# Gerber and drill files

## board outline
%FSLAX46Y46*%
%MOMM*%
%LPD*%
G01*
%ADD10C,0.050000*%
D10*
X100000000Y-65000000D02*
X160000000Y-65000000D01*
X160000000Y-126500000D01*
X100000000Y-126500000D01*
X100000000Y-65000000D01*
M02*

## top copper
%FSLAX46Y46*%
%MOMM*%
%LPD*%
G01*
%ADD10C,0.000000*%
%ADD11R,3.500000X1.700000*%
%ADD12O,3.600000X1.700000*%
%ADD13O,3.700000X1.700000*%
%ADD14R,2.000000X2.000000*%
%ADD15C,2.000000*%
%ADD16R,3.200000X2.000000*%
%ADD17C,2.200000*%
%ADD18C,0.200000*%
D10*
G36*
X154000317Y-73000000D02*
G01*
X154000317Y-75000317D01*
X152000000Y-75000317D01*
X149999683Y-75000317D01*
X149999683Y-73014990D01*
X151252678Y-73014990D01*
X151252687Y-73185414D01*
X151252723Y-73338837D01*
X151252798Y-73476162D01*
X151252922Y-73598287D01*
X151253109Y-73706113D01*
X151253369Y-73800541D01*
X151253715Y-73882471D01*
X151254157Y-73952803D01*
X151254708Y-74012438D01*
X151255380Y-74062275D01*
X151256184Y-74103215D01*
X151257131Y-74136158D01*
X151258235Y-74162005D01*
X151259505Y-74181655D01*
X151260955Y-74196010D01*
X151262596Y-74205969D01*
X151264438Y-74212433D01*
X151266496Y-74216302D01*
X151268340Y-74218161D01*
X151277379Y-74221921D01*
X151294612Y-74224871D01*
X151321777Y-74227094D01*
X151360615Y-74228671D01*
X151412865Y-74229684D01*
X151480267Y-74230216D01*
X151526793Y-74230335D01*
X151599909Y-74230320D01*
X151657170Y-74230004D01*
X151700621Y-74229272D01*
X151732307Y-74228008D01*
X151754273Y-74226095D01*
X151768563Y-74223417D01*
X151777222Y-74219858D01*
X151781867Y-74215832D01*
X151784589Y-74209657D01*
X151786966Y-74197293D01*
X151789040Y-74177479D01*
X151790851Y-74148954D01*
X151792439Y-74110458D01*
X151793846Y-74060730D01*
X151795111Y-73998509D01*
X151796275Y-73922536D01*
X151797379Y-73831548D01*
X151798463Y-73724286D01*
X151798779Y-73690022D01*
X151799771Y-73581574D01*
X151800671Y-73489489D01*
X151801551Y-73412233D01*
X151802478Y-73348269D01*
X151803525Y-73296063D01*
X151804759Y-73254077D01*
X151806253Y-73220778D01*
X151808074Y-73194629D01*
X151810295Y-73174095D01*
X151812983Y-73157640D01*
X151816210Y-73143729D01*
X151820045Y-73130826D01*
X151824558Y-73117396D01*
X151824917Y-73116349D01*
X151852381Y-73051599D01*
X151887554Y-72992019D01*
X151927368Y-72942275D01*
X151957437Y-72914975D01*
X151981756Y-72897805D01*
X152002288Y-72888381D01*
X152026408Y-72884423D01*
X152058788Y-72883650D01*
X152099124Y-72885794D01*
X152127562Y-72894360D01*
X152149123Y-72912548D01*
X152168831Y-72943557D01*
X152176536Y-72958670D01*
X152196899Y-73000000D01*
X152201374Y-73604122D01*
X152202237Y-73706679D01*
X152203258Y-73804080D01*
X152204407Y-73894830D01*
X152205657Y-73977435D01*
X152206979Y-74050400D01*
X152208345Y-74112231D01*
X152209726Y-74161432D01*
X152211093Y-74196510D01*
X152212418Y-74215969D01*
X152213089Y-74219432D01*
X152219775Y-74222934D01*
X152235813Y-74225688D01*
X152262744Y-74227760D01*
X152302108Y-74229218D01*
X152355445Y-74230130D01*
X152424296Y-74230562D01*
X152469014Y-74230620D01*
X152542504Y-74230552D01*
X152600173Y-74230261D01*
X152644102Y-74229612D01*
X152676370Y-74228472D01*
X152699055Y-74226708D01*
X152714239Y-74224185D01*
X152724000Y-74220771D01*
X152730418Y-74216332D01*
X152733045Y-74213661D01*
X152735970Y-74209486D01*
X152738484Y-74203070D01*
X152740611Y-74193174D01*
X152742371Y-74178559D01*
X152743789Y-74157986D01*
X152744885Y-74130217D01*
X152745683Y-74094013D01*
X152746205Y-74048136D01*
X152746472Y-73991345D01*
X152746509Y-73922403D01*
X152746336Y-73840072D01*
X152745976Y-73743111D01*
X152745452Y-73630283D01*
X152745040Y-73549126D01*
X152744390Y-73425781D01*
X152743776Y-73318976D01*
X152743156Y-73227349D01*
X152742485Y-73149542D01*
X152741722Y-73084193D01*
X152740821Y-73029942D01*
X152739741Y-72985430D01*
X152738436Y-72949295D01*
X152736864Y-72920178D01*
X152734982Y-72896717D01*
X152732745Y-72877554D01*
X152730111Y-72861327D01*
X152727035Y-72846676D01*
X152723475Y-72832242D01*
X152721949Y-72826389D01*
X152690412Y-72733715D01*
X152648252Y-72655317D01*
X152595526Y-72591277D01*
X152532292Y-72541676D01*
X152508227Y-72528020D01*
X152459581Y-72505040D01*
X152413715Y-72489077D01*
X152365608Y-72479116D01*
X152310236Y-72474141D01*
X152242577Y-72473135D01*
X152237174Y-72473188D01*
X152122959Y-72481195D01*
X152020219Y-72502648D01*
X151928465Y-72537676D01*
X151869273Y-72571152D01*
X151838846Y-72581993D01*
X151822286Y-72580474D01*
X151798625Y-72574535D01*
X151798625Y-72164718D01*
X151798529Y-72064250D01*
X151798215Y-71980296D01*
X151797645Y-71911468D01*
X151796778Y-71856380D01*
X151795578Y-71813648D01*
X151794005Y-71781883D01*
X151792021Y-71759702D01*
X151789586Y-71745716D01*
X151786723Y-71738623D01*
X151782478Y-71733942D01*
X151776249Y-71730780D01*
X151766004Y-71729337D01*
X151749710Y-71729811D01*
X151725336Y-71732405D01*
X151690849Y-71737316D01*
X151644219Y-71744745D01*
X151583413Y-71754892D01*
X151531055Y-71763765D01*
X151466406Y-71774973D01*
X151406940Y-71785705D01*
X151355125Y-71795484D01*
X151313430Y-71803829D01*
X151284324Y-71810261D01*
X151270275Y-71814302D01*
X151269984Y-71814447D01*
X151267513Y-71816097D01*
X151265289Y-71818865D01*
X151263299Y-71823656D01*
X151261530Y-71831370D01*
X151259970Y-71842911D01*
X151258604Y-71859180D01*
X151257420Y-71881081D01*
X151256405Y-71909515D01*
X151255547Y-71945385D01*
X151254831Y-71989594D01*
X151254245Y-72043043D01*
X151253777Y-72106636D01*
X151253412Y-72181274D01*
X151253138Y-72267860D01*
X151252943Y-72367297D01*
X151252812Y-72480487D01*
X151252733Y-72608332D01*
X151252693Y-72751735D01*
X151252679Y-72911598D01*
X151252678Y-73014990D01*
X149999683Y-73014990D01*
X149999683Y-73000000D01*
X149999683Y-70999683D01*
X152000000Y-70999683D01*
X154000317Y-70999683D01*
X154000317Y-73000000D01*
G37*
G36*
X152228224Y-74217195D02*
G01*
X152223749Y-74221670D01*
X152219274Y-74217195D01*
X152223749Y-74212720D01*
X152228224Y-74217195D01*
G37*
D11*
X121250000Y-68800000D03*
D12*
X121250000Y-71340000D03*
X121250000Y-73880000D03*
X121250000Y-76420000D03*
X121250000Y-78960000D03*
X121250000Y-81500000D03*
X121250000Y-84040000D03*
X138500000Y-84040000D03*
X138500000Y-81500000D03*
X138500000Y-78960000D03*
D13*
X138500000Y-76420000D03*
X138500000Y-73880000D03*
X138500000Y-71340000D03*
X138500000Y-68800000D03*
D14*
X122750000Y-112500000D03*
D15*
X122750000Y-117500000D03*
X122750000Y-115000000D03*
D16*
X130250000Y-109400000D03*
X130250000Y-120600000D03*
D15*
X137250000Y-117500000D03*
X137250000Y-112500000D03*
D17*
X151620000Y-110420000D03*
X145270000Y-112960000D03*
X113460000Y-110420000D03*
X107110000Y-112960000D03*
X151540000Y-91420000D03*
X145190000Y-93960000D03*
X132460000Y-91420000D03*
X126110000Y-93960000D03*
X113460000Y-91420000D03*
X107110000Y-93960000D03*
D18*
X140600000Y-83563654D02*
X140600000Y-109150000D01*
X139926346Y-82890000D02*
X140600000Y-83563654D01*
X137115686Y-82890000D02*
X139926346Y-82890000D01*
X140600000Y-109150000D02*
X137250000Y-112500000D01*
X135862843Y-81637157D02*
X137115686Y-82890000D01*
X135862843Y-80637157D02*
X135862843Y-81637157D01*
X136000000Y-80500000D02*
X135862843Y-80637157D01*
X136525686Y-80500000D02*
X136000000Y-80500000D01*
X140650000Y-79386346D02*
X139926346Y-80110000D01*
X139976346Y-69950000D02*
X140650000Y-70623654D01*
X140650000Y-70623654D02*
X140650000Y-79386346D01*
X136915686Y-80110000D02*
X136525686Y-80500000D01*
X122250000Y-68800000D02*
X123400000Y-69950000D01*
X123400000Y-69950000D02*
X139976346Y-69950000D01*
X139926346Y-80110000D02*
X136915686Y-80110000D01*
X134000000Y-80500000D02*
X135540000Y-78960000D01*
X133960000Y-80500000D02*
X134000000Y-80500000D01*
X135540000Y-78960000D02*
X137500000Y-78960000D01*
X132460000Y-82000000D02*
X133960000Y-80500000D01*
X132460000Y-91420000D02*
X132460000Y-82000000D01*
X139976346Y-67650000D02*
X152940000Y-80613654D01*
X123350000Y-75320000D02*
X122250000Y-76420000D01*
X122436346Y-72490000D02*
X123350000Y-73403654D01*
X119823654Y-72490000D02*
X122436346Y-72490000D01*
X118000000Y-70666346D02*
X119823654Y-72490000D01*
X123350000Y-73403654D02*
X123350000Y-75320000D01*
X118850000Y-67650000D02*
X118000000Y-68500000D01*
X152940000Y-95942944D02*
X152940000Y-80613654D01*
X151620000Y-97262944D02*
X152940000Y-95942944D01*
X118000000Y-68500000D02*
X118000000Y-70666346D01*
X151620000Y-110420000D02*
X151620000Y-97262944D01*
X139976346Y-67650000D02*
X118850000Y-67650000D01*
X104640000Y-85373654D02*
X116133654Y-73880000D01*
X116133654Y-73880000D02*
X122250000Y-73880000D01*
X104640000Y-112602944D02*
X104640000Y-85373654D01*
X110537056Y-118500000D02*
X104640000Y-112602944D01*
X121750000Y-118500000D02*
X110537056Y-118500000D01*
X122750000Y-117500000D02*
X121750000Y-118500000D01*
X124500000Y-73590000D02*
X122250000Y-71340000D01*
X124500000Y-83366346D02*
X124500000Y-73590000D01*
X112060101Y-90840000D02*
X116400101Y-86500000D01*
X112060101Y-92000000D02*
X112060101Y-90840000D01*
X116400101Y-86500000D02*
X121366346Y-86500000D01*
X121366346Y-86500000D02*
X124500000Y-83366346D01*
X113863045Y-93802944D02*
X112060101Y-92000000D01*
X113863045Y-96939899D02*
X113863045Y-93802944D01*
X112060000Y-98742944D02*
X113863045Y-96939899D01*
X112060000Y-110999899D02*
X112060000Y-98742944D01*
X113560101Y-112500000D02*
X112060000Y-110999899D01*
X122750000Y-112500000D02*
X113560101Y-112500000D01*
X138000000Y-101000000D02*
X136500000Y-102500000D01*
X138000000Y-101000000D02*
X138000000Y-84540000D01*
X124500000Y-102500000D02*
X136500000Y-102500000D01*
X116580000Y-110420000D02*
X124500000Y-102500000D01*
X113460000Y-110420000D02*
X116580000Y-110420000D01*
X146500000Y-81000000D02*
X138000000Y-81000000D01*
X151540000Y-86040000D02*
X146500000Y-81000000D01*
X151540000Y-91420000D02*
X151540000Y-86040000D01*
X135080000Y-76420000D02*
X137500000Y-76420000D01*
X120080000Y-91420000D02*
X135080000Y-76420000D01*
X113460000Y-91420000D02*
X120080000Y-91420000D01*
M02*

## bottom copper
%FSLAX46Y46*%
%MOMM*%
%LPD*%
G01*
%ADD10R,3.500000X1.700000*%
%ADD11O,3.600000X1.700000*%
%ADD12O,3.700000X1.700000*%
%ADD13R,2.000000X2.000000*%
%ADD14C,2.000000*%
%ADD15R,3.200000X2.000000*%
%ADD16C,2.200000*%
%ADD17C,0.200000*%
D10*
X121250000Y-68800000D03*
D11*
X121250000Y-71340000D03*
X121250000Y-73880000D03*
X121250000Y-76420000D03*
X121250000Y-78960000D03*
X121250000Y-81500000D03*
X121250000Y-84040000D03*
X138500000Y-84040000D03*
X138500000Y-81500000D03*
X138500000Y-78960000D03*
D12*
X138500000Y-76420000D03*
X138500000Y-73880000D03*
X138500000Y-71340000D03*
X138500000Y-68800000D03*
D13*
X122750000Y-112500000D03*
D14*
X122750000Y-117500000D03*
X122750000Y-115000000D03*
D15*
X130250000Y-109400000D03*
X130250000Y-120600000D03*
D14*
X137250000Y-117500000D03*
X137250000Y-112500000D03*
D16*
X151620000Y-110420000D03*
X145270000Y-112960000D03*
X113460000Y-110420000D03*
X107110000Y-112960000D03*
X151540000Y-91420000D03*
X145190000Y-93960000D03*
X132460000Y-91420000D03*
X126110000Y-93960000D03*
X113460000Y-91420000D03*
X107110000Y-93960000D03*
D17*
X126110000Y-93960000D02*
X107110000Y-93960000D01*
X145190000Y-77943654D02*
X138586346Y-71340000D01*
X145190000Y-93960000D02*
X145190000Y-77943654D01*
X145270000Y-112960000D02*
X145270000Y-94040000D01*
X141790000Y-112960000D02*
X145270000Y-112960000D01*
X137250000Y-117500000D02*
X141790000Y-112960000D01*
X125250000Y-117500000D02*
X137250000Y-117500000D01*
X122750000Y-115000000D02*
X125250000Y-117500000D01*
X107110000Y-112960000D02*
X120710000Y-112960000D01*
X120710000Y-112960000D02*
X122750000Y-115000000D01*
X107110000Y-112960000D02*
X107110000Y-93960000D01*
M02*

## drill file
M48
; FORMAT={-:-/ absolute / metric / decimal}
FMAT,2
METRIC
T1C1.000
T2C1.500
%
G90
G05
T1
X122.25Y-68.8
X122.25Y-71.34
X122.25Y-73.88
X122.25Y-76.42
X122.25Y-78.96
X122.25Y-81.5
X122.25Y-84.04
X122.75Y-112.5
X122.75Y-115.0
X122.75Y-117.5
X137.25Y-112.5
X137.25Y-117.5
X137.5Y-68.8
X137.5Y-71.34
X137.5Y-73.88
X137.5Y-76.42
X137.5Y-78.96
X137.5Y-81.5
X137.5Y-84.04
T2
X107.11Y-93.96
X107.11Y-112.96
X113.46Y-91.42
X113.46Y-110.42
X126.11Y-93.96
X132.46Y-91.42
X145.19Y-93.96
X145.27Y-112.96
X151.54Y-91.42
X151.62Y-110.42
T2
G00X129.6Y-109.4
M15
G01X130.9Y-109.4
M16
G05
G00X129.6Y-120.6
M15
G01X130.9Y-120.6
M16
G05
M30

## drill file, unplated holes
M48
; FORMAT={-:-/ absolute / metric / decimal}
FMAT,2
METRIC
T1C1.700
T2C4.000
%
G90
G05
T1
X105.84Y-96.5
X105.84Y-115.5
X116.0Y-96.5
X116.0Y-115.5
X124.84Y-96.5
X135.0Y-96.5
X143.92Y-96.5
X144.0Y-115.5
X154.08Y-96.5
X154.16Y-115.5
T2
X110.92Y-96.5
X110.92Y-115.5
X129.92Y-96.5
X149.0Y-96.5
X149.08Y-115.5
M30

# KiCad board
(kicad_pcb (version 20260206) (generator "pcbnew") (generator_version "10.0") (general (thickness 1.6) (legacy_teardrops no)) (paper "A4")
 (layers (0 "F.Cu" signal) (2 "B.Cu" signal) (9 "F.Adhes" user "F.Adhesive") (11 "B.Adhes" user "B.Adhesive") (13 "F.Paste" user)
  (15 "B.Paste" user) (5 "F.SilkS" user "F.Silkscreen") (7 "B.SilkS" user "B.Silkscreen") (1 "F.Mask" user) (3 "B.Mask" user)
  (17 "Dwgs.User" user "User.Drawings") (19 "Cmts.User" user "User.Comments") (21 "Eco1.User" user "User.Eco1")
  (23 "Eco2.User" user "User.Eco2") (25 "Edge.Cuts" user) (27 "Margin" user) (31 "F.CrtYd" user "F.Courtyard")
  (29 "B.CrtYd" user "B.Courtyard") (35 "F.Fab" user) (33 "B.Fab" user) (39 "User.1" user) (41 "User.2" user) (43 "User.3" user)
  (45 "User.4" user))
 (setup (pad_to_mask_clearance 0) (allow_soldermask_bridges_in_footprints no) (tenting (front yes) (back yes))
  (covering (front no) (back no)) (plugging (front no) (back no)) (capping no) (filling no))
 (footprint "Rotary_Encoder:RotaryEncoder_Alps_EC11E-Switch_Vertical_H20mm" (layer "F.Cu") (at 122.75 112.5)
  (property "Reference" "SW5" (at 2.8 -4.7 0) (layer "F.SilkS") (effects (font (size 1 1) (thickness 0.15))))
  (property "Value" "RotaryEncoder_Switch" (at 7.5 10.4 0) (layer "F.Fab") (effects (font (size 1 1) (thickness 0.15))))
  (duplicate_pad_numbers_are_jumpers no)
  (pad "A" thru_hole rect (at 0 0) (size 2 2) (drill 1) (layers "*.Cu" "*.Mask") (remove_unused_layers no) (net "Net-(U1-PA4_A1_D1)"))
  (pad "B" thru_hole circle (at 0 5) (size 2 2) (drill 1) (layers "*.Cu" "*.Mask") (remove_unused_layers no) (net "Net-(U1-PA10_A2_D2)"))
  (pad "C" thru_hole circle (at 0 2.5) (size 2 2) (drill 1) (layers "*.Cu" "*.Mask") (remove_unused_layers no) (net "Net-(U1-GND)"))
  (pad "MP" thru_hole rect (at 7.5 -3.1) (size 3.2 2) (drill oval 2.8 1.5) (layers "*.Cu" "*.Mask") (remove_unused_layers no))
  (pad "MP" thru_hole rect (at 7.5 8.1) (size 3.2 2) (drill oval 2.8 1.5) (layers "*.Cu" "*.Mask") (remove_unused_layers no))
  (pad "S1" thru_hole circle (at 14.5 5) (size 2 2) (drill 1) (layers "*.Cu" "*.Mask") (remove_unused_layers no) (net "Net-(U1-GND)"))
  (pad "S2" thru_hole circle (at 14.5 0) (size 2 2) (drill 1) (layers "*.Cu" "*.Mask") (remove_unused_layers no) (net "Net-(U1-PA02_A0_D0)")))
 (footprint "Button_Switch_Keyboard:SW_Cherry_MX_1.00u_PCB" (layer "F.Cu") (at 113.46 110.42)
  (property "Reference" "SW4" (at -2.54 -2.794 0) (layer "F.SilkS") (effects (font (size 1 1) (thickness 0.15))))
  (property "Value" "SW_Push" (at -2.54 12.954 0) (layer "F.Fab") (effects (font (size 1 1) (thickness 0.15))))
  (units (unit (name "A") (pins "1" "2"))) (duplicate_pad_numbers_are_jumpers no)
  (pad "" np_thru_hole circle (at -7.62 5.08) (size 1.7 1.7) (drill 1.7) (layers "*.Cu" "*.Mask"))
  (pad "" np_thru_hole circle (at -2.54 5.08) (size 4 4) (drill 4) (layers "*.Cu" "*.Mask"))
  (pad "" np_thru_hole circle (at 2.54 5.08) (size 1.7 1.7) (drill 1.7) (layers "*.Cu" "*.Mask"))
  (pad "1" thru_hole circle (at 0 0) (size 2.2 2.2) (drill 1.5) (layers "*.Cu" "*.Mask") (remove_unused_layers no)
   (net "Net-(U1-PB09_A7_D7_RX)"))
  (pad "2" thru_hole circle (at -6.35 2.54) (size 2.2 2.2) (drill 1.5) (layers "*.Cu" "*.Mask") (remove_unused_layers no)
   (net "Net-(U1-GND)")))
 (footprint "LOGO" (layer "F.Cu") (at 152 73)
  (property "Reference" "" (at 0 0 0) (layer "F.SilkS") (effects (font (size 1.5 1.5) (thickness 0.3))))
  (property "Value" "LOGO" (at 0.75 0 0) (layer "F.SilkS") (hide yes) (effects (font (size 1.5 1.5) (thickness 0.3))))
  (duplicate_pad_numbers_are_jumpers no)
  (fp_poly
   (pts (xy 0.228224 1.217195) (xy 0.223749 1.22167) (xy 0.219274 1.217195) (xy 0.223749 1.21272)) (stroke (width 0) (type solid))
   (fill yes) (layer "F.Cu"))
  (fp_poly
   (pts (xy 2.000317 0) (xy 2.000317 2.000317) (xy 0 2.000317) (xy -2.000317 2.000317) (xy -2.000317 0.01499) (xy -0.747322 0.01499)
    (xy -0.747313 0.185414) (xy -0.747277 0.338837) (xy -0.747202 0.476162) (xy -0.747078 0.598287) (xy -0.746891 0.706113)
    (xy -0.746631 0.800541) (xy -0.746285 0.882471) (xy -0.745843 0.952803) (xy -0.745292 1.012438) (xy -0.74462 1.062275)
    (xy -0.743816 1.103215) (xy -0.742869 1.136158) (xy -0.741765 1.162005) (xy -0.740495 1.181655) (xy -0.739045 1.19601)
    (xy -0.737404 1.205969) (xy -0.735562 1.212433) (xy -0.733504 1.216302) (xy -0.73166 1.218161) (xy -0.722621 1.221921)
    (xy -0.705388 1.224871) (xy -0.678223 1.227094) (xy -0.639385 1.228671) (xy -0.587135 1.229684) (xy -0.519733 1.230216)
    (xy -0.473207 1.230335) (xy -0.400091 1.23032) (xy -0.34283 1.230004) (xy -0.299379 1.229272) (xy -0.267693 1.228008)
    (xy -0.245727 1.226095) (xy -0.231437 1.223417) (xy -0.222778 1.219858) (xy -0.218133 1.215832) (xy -0.215411 1.209657)
    (xy -0.213034 1.197293) (xy -0.21096 1.177479) (xy -0.209149 1.148954) (xy -0.207561 1.110458) (xy -0.206154 1.06073)
    (xy -0.204889 0.998509) (xy -0.203725 0.922536) (xy -0.202621 0.831548) (xy -0.201537 0.724286) (xy -0.201221 0.690022)
    (xy -0.200229 0.581574) (xy -0.199329 0.489489) (xy -0.198449 0.412233) (xy -0.197522 0.348269) (xy -0.196475 0.296063)
    (xy -0.195241 0.254077) (xy -0.193747 0.220778) (xy -0.191926 0.194629) (xy -0.189705 0.174095) (xy -0.187017 0.15764)
    (xy -0.18379 0.143729) (xy -0.179955 0.130826) (xy -0.175442 0.117396) (xy -0.175083 0.116349) (xy -0.147619 0.051599)
    (xy -0.112446 -0.007981) (xy -0.072632 -0.057725) (xy -0.042563 -0.085025) (xy -0.018244 -0.102195) (xy 0.002288 -0.111619)
    (xy 0.026408 -0.115577) (xy 0.058788 -0.11635) (xy 0.099124 -0.114206) (xy 0.127562 -0.10564) (xy 0.149123 -0.087452)
    (xy 0.168831 -0.056443) (xy 0.176536 -0.04133) (xy 0.196899 0) (xy 0.201374 0.604122) (xy 0.202237 0.706679) (xy 0.203258 0.80408)
    (xy 0.204407 0.89483) (xy 0.205657 0.977435) (xy 0.206979 1.0504) (xy 0.208345 1.112231) (xy 0.209726 1.161432) (xy 0.211093 1.19651)
    (xy 0.212418 1.215969) (xy 0.213089 1.219432) (xy 0.219775 1.222934) (xy 0.235813 1.225688) (xy 0.262744 1.22776) (xy 0.302108 1.229218)
    (xy 0.355445 1.23013) (xy 0.424296 1.230562) (xy 0.469014 1.23062) (xy 0.542504 1.230552) (xy 0.600173 1.230261) (xy 0.644102 1.229612)
    (xy 0.67637 1.228472) (xy 0.699055 1.226708) (xy 0.714239 1.224185) (xy 0.724 1.220771) (xy 0.730418 1.216332) (xy 0.733045 1.213661)
    (xy 0.73597 1.209486) (xy 0.738484 1.20307) (xy 0.740611 1.193174) (xy 0.742371 1.178559) (xy 0.743789 1.157986) (xy 0.744885 1.130217)
    (xy 0.745683 1.094013) (xy 0.746205 1.048136) (xy 0.746472 0.991345) (xy 0.746509 0.922403) (xy 0.746336 0.840072)
    (xy 0.745976 0.743111) (xy 0.745452 0.630283) (xy 0.74504 0.549126) (xy 0.74439 0.425781) (xy 0.743776 0.318976) (xy 0.743156 0.227349)
    (xy 0.742485 0.149542) (xy 0.741722 0.084193) (xy 0.740821 0.029942) (xy 0.739741 -0.01457) (xy 0.738436 -0.050705)
    (xy 0.736864 -0.079822) (xy 0.734982 -0.103283) (xy 0.732745 -0.122446) (xy 0.730111 -0.138673) (xy 0.727035 -0.153324)
    (xy 0.723475 -0.167758) (xy 0.721949 -0.173611) (xy 0.690412 -0.266285) (xy 0.648252 -0.344683) (xy 0.595526 -0.408723)
    (xy 0.532292 -0.458324) (xy 0.508227 -0.47198) (xy 0.459581 -0.49496) (xy 0.413715 -0.510923) (xy 0.365608 -0.520884)
    (xy 0.310236 -0.525859) (xy 0.242577 -0.526865) (xy 0.237174 -0.526812) (xy 0.122959 -0.518805) (xy 0.020219 -0.497352)
    (xy -0.071535 -0.462324) (xy -0.130727 -0.428848) (xy -0.161154 -0.418007) (xy -0.177714 -0.419526) (xy -0.201375 -0.425465)
    (xy -0.201375 -0.835282) (xy -0.201471 -0.93575) (xy -0.201785 -1.019704) (xy -0.202355 -1.088532) (xy -0.203222 -1.14362)
    (xy -0.204422 -1.186352) (xy -0.205995 -1.218117) (xy -0.207979 -1.240298) (xy -0.210414 -1.254284) (xy -0.213277 -1.261377)
    (xy -0.217522 -1.266058) (xy -0.223751 -1.26922) (xy -0.233996 -1.270663) (xy -0.25029 -1.270189) (xy -0.274664 -1.267595)
    (xy -0.309151 -1.262684) (xy -0.355781 -1.255255) (xy -0.416587 -1.245108) (xy -0.468945 -1.236235) (xy -0.533594 -1.225027)
    (xy -0.59306 -1.214295) (xy -0.644875 -1.204516) (xy -0.68657 -1.196171) (xy -0.715676 -1.189739) (xy -0.729725 -1.185698)
    (xy -0.730016 -1.185553) (xy -0.732487 -1.183903) (xy -0.734711 -1.181135) (xy -0.736701 -1.176344) (xy -0.73847 -1.16863)
    (xy -0.74003 -1.157089) (xy -0.741396 -1.14082) (xy -0.74258 -1.118919) (xy -0.743595 -1.090485) (xy -0.744453 -1.054615)
    (xy -0.745169 -1.010406) (xy -0.745755 -0.956957) (xy -0.746223 -0.893364) (xy -0.746588 -0.818726) (xy -0.746862 -0.73214)
    (xy -0.747057 -0.632703) (xy -0.747188 -0.519513) (xy -0.747267 -0.391668) (xy -0.747307 -0.248265) (xy -0.747321 -0.088402)
    (xy -0.747322 0.01499) (xy -2.000317 0.01499) (xy -2.000317 0) (xy -2.000317 -2.000317) (xy 0 -2.000317) (xy 2.000317 -2.000317))
   (stroke (width 0) (type solid)) (fill yes) (layer "F.Cu")))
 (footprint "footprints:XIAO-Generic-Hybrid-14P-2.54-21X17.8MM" (layer "F.Cu") (at 129.875 76.42)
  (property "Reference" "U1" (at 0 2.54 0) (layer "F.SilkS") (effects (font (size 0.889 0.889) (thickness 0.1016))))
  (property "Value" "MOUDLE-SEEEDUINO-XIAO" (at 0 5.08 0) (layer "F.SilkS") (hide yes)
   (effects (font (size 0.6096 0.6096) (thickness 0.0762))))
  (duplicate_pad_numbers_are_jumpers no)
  (pad "1" thru_hole rect (at -7.625 -7.62) (size 3.5 1.7) (drill 1 (offset -1 0)) (layers "*.Cu" "*.Mask") (remove_unused_layers no)
   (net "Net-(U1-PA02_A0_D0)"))
  (pad "2" thru_hole oval (at -7.625 -5.08) (size 3.6 1.7) (drill 1 (offset -1 0)) (layers "*.Cu" "*.Mask") (remove_unused_layers no)
   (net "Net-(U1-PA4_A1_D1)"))
  (pad "3" thru_hole oval (at -7.625 -2.54) (size 3.6 1.7) (drill 1 (offset -1 0)) (layers "*.Cu" "*.Mask") (remove_unused_layers no)
   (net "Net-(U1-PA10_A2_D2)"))
  (pad "4" thru_hole oval (at -7.625 0) (size 3.6 1.7) (drill 1 (offset -1 0)) (layers "*.Cu" "*.Mask") (remove_unused_layers no)
   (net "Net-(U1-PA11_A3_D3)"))
  (pad "5" thru_hole oval (at -7.625 2.54) (size 3.6 1.7) (drill 1 (offset -1 0)) (layers "*.Cu" "*.Mask") (remove_unused_layers no)
   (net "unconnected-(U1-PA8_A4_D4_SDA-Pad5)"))
  (pad "6" thru_hole oval (at -7.625 5.08 180) (size 3.6 1.7) (drill 1 (offset 1 0)) (layers "*.Cu" "*.Mask") (remove_unused_layers no)
   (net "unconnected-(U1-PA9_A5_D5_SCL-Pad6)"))
  (pad "7" thru_hole oval (at -7.625 7.62) (size 3.6 1.7) (drill 1 (offset -1 0)) (layers "*.Cu" "*.Mask") (remove_unused_layers no)
   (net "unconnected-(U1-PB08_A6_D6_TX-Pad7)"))
  (pad "8" thru_hole oval (at 7.625 7.62) (size 3.6 1.7) (drill 1 (offset 1 0)) (layers "*.Cu" "*.Mask") (remove_unused_layers no)
   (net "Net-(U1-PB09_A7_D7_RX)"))
  (pad "9" thru_hole oval (at 7.625 5.08) (size 3.6 1.7) (drill 1 (offset 1 0)) (layers "*.Cu" "*.Mask") (remove_unused_layers no)
   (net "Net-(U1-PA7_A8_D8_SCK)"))
  (pad "10" thru_hole oval (at 7.625 2.54) (size 3.6 1.7) (drill 1 (offset 1 0)) (layers "*.Cu" "*.Mask") (remove_unused_layers no)
   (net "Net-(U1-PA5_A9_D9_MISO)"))
  (pad "11" thru_hole oval (at 7.625 0) (size 3.7 1.7) (drill 1 (offset 1 0)) (layers "*.Cu" "*.Mask") (remove_unused_layers no)
   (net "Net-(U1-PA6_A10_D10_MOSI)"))
  (pad "12" thru_hole oval (at 7.625 -2.54) (size 3.7 1.7) (drill 1 (offset 1 0)) (layers "*.Cu" "*.Mask") (remove_unused_layers no)
   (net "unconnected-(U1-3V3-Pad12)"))
  (pad "13" thru_hole oval (at 7.625 -5.08) (size 3.7 1.7) (drill 1 (offset 1 0)) (layers "*.Cu" "*.Mask") (remove_unused_layers no)
   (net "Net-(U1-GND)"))
  (pad "14" thru_hole oval (at 7.625 -7.62) (size 3.7 1.7) (drill 1 (offset 1 0)) (layers "*.Cu" "*.Mask") (remove_unused_layers no)
   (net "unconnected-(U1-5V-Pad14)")))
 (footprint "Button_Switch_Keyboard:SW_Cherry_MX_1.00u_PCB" (layer "F.Cu") (at 113.46 91.42)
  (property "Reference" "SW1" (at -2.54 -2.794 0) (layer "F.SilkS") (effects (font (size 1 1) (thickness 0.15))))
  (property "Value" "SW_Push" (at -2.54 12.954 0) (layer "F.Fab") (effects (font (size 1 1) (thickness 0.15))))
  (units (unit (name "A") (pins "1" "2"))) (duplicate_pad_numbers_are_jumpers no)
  (pad "" np_thru_hole circle (at -7.62 5.08) (size 1.7 1.7) (drill 1.7) (layers "*.Cu" "*.Mask"))
  (pad "" np_thru_hole circle (at -2.54 5.08) (size 4 4) (drill 4) (layers "*.Cu" "*.Mask"))
  (pad "" np_thru_hole circle (at 2.54 5.08) (size 1.7 1.7) (drill 1.7) (layers "*.Cu" "*.Mask"))
  (pad "1" thru_hole circle (at 0 0) (size 2.2 2.2) (drill 1.5) (layers "*.Cu" "*.Mask") (remove_unused_layers no)
   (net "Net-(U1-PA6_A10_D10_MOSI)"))
  (pad "2" thru_hole circle (at -6.35 2.54) (size 2.2 2.2) (drill 1.5) (layers "*.Cu" "*.Mask") (remove_unused_layers no)
   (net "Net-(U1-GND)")))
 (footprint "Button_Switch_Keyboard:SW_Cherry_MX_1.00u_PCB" (layer "F.Cu") (at 151.62 110.42)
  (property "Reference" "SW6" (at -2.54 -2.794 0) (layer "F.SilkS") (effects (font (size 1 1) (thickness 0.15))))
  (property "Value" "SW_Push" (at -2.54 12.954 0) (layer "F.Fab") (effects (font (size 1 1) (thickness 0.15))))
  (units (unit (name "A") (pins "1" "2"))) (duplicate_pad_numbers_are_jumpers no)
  (pad "" np_thru_hole circle (at -7.62 5.08) (size 1.7 1.7) (drill 1.7) (layers "*.Cu" "*.Mask"))
  (pad "" np_thru_hole circle (at -2.54 5.08) (size 4 4) (drill 4) (layers "*.Cu" "*.Mask"))
  (pad "" np_thru_hole circle (at 2.54 5.08) (size 1.7 1.7) (drill 1.7) (layers "*.Cu" "*.Mask"))
  (pad "1" thru_hole circle (at 0 0) (size 2.2 2.2) (drill 1.5) (layers "*.Cu" "*.Mask") (remove_unused_layers no)
   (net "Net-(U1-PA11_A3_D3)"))
  (pad "2" thru_hole circle (at -6.35 2.54) (size 2.2 2.2) (drill 1.5) (layers "*.Cu" "*.Mask") (remove_unused_layers no)
   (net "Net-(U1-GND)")))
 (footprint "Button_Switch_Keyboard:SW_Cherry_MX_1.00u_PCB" (layer "F.Cu") (at 151.54 91.42)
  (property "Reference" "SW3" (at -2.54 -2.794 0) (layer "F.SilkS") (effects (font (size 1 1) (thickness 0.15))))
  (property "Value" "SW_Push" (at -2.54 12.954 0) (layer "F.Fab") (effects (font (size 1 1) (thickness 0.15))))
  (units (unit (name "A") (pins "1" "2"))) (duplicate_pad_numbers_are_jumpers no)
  (pad "" np_thru_hole circle (at -7.62 5.08) (size 1.7 1.7) (drill 1.7) (layers "*.Cu" "*.Mask"))
  (pad "" np_thru_hole circle (at -2.54 5.08) (size 4 4) (drill 4) (layers "*.Cu" "*.Mask"))
  (pad "" np_thru_hole circle (at 2.54 5.08) (size 1.7 1.7) (drill 1.7) (layers "*.Cu" "*.Mask"))
  (pad "1" thru_hole circle (at 0 0) (size 2.2 2.2) (drill 1.5) (layers "*.Cu" "*.Mask") (remove_unused_layers no)
   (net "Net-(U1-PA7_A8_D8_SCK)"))
  (pad "2" thru_hole circle (at -6.35 2.54) (size 2.2 2.2) (drill 1.5) (layers "*.Cu" "*.Mask") (remove_unused_layers no)
   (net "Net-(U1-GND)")))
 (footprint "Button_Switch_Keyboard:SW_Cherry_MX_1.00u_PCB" (layer "F.Cu") (at 132.46 91.42)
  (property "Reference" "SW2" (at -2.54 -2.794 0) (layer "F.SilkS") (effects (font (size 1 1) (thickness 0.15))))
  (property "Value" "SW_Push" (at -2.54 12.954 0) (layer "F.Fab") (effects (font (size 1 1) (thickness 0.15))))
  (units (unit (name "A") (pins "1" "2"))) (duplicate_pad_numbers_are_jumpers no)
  (pad "" np_thru_hole circle (at -7.62 5.08) (size 1.7 1.7) (drill 1.7) (layers "*.Cu" "*.Mask"))
  (pad "" np_thru_hole circle (at -2.54 5.08) (size 4 4) (drill 4) (layers "*.Cu" "*.Mask"))
  (pad "" np_thru_hole circle (at 2.54 5.08) (size 1.7 1.7) (drill 1.7) (layers "*.Cu" "*.Mask"))
  (pad "1" thru_hole circle (at 0 0) (size 2.2 2.2) (drill 1.5) (layers "*.Cu" "*.Mask") (remove_unused_layers no)
   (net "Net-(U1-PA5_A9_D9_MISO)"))
  (pad "2" thru_hole circle (at -6.35 2.54) (size 2.2 2.2) (drill 1.5) (layers "*.Cu" "*.Mask") (remove_unused_layers no)
   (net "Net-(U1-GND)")))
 (gr_rect (start 100 65) (end 160 126.5) (stroke (width 0.05) (type default)) (fill no) (layer "Edge.Cuts"))
 (segment (start 145.27 112.96) (end 145.27 94.04) (width 0.2) (layer "B.Cu") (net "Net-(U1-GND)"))
 (segment (start 126.11 93.96) (end 107.11 93.96) (width 0.2) (layer "B.Cu") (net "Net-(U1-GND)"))
 (segment (start 145.19 77.943654) (end 138.586346 71.34) (width 0.2) (layer "B.Cu") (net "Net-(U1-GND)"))
 (segment (start 141.79 112.96) (end 145.27 112.96) (width 0.2) (layer "B.Cu") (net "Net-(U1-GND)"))
 (segment (start 120.71 112.96) (end 122.75 115) (width 0.2) (layer "B.Cu") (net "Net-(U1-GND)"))
 (segment (start 107.11 112.96) (end 120.71 112.96) (width 0.2) (layer "B.Cu") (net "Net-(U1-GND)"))
 (segment (start 107.11 112.96) (end 107.11 93.96) (width 0.2) (layer "B.Cu") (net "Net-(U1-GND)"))
 (segment (start 122.75 115) (end 125.25 117.5) (width 0.2) (layer "B.Cu") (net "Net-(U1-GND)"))
 (segment (start 137.25 117.5) (end 141.79 112.96) (width 0.2) (layer "B.Cu") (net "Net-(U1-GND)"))
 (segment (start 125.25 117.5) (end 137.25 117.5) (width 0.2) (layer "B.Cu") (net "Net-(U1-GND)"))
 (segment (start 145.19 93.96) (end 145.19 77.943654) (width 0.2) (layer "B.Cu") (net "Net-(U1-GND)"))
 (segment (start 135.08 76.42) (end 137.5 76.42) (width 0.2) (layer "F.Cu") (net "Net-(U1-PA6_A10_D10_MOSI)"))
 (segment (start 113.46 91.42) (end 120.08 91.42) (width 0.2) (layer "F.Cu") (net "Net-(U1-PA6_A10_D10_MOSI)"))
 (segment (start 120.08 91.42) (end 135.08 76.42) (width 0.2) (layer "F.Cu") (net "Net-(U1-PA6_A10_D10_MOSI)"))
 (segment (start 133.96 80.5) (end 134 80.5) (width 0.2) (layer "F.Cu") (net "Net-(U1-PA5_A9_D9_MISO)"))
 (segment (start 132.46 82) (end 133.96 80.5) (width 0.2) (layer "F.Cu") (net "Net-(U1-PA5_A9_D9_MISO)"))
 (segment (start 134 80.5) (end 135.54 78.96) (width 0.2) (layer "F.Cu") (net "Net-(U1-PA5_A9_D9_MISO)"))
 (segment (start 132.46 91.42) (end 132.46 82) (width 0.2) (layer "F.Cu") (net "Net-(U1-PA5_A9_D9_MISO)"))
 (segment (start 135.54 78.96) (end 137.5 78.96) (width 0.2) (layer "F.Cu") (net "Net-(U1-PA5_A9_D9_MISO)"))
 (segment (start 146.5 81) (end 138 81) (width 0.2) (layer "F.Cu") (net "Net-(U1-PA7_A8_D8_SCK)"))
 (segment (start 151.54 86.04) (end 146.5 81) (width 0.2) (layer "F.Cu") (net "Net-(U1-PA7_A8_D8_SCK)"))
 (segment (start 151.54 91.42) (end 151.54 86.04) (width 0.2) (layer "F.Cu") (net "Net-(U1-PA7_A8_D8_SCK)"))
 (segment (start 116.58 110.42) (end 124.5 102.5) (width 0.2) (layer "F.Cu") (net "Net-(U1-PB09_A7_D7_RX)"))
 (segment (start 124.5 102.5) (end 136.5 102.5) (width 0.2) (layer "F.Cu") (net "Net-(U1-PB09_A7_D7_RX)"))
 (segment (start 138 101) (end 136.5 102.5) (width 0.2) (layer "F.Cu") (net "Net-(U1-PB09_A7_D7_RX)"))
 (segment (start 113.46 110.42) (end 116.58 110.42) (width 0.2) (layer "F.Cu") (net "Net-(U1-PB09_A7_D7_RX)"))
 (segment (start 138 101) (end 138 84.54) (width 0.2) (layer "F.Cu") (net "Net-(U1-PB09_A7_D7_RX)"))
 (segment (start 112.060101 92) (end 112.060101 90.84) (width 0.2) (layer "F.Cu") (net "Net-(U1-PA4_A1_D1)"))
 (segment (start 124.5 83.366346) (end 124.5 73.59) (width 0.2) (layer "F.Cu") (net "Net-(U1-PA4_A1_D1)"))
 (segment (start 112.06 98.742944) (end 113.863045 96.939899) (width 0.2) (layer "F.Cu") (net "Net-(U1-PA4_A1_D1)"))
 (segment (start 113.863045 96.939899) (end 113.863045 93.802944) (width 0.2) (layer "F.Cu") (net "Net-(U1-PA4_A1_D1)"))
 (segment (start 124.5 73.59) (end 122.25 71.34) (width 0.2) (layer "F.Cu") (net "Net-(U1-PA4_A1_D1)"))
 (segment (start 112.060101 90.84) (end 116.400101 86.5) (width 0.2) (layer "F.Cu") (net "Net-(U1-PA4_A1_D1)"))
 (segment (start 116.400101 86.5) (end 121.366346 86.5) (width 0.2) (layer "F.Cu") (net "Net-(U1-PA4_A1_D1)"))
 (segment (start 122.75 112.5) (end 113.560101 112.5) (width 0.2) (layer "F.Cu") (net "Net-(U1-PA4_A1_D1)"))
 (segment (start 113.560101 112.5) (end 112.06 110.999899) (width 0.2) (layer "F.Cu") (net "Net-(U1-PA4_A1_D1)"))
 (segment (start 112.06 110.999899) (end 112.06 98.742944) (width 0.2) (layer "F.Cu") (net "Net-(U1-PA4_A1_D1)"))
 (segment (start 113.863045 93.802944) (end 112.060101 92) (width 0.2) (layer "F.Cu") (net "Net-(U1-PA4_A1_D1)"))
 (segment (start 121.366346 86.5) (end 124.5 83.366346) (width 0.2) (layer "F.Cu") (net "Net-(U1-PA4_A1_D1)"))
 (segment (start 122.25 68.8) (end 123.4 69.95) (width 0.2) (layer "F.Cu") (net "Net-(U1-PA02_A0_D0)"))
 (segment (start 135.862843 80.637157) (end 135.862843 81.637157) (width 0.2) (layer "F.Cu") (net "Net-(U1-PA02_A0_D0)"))
 (segment (start 137.115686 82.89) (end 139.926346 82.89) (width 0.2) (layer "F.Cu") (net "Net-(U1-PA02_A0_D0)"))
 (segment (start 140.6 109.15) (end 137.25 112.5) (width 0.2) (layer "F.Cu") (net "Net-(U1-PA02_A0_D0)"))
 (segment (start 139.926346 82.89) (end 140.6 83.563654) (width 0.2) (layer "F.Cu") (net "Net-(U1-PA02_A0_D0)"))
 (segment (start 140.65 70.623654) (end 140.65 79.386346) (width 0.2) (layer "F.Cu") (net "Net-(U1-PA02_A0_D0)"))
 (segment (start 139.926346 80.11) (end 136.915686 80.11) (width 0.2) (layer "F.Cu") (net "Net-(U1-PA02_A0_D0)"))
 (segment (start 123.4 69.95) (end 139.976346 69.95) (width 0.2) (layer "F.Cu") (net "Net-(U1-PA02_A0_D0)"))
 (segment (start 140.6 83.563654) (end 140.6 109.15) (width 0.2) (layer "F.Cu") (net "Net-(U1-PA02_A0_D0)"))
 (segment (start 136.915686 80.11) (end 136.525686 80.5) (width 0.2) (layer "F.Cu") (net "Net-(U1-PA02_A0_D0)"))
 (segment (start 136 80.5) (end 135.862843 80.637157) (width 0.2) (layer "F.Cu") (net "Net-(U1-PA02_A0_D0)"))
 (segment (start 139.976346 69.95) (end 140.65 70.623654) (width 0.2) (layer "F.Cu") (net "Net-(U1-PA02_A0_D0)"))
 (segment (start 135.862843 81.637157) (end 137.115686 82.89) (width 0.2) (layer "F.Cu") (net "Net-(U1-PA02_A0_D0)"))
 (segment (start 136.525686 80.5) (end 136 80.5) (width 0.2) (layer "F.Cu") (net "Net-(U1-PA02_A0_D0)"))
 (segment (start 140.65 79.386346) (end 139.926346 80.11) (width 0.2) (layer "F.Cu") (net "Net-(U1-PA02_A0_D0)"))
 (segment (start 121.75 118.5) (end 110.537056 118.5) (width 0.2) (layer "F.Cu") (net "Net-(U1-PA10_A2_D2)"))
 (segment (start 122.75 117.5) (end 121.75 118.5) (width 0.2) (layer "F.Cu") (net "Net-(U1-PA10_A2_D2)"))
 (segment (start 104.64 112.602944) (end 104.64 85.373654) (width 0.2) (layer "F.Cu") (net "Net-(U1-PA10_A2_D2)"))
 (segment (start 104.64 85.373654) (end 116.133654 73.88) (width 0.2) (layer "F.Cu") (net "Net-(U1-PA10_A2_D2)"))
 (segment (start 110.537056 118.5) (end 104.64 112.602944) (width 0.2) (layer "F.Cu") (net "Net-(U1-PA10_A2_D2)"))
 (segment (start 116.133654 73.88) (end 122.25 73.88) (width 0.2) (layer "F.Cu") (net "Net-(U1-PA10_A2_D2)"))
 (segment (start 123.35 75.32) (end 122.25 76.42) (width 0.2) (layer "F.Cu") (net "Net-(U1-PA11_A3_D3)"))
 (segment (start 118 70.666346) (end 119.823654 72.49) (width 0.2) (layer "F.Cu") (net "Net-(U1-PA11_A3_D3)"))
 (segment (start 139.976346 67.65) (end 152.94 80.613654) (width 0.2) (layer "F.Cu") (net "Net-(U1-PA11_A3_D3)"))
 (segment (start 118.85 67.65) (end 118 68.5) (width 0.2) (layer "F.Cu") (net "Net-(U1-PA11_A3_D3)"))
 (segment (start 118 68.5) (end 118 70.666346) (width 0.2) (layer "F.Cu") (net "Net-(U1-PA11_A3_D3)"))
 (segment (start 139.976346 67.65) (end 118.85 67.65) (width 0.2) (layer "F.Cu") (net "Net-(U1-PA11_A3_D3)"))
 (segment (start 119.823654 72.49) (end 122.436346 72.49) (width 0.2) (layer "F.Cu") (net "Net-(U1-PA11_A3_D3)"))
 (segment (start 151.62 97.262944) (end 152.94 95.942944) (width 0.2) (layer "F.Cu") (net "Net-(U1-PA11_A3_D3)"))
 (segment (start 123.35 73.403654) (end 123.35 75.32) (width 0.2) (layer "F.Cu") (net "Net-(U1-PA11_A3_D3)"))
 (segment (start 151.62 110.42) (end 151.62 97.262944) (width 0.2) (layer "F.Cu") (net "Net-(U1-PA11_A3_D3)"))
 (segment (start 152.94 95.942944) (end 152.94 80.613654) (width 0.2) (layer "F.Cu") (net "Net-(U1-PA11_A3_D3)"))
 (segment (start 122.436346 72.49) (end 123.35 73.403654) (width 0.2) (layer "F.Cu") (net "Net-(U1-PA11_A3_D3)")))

